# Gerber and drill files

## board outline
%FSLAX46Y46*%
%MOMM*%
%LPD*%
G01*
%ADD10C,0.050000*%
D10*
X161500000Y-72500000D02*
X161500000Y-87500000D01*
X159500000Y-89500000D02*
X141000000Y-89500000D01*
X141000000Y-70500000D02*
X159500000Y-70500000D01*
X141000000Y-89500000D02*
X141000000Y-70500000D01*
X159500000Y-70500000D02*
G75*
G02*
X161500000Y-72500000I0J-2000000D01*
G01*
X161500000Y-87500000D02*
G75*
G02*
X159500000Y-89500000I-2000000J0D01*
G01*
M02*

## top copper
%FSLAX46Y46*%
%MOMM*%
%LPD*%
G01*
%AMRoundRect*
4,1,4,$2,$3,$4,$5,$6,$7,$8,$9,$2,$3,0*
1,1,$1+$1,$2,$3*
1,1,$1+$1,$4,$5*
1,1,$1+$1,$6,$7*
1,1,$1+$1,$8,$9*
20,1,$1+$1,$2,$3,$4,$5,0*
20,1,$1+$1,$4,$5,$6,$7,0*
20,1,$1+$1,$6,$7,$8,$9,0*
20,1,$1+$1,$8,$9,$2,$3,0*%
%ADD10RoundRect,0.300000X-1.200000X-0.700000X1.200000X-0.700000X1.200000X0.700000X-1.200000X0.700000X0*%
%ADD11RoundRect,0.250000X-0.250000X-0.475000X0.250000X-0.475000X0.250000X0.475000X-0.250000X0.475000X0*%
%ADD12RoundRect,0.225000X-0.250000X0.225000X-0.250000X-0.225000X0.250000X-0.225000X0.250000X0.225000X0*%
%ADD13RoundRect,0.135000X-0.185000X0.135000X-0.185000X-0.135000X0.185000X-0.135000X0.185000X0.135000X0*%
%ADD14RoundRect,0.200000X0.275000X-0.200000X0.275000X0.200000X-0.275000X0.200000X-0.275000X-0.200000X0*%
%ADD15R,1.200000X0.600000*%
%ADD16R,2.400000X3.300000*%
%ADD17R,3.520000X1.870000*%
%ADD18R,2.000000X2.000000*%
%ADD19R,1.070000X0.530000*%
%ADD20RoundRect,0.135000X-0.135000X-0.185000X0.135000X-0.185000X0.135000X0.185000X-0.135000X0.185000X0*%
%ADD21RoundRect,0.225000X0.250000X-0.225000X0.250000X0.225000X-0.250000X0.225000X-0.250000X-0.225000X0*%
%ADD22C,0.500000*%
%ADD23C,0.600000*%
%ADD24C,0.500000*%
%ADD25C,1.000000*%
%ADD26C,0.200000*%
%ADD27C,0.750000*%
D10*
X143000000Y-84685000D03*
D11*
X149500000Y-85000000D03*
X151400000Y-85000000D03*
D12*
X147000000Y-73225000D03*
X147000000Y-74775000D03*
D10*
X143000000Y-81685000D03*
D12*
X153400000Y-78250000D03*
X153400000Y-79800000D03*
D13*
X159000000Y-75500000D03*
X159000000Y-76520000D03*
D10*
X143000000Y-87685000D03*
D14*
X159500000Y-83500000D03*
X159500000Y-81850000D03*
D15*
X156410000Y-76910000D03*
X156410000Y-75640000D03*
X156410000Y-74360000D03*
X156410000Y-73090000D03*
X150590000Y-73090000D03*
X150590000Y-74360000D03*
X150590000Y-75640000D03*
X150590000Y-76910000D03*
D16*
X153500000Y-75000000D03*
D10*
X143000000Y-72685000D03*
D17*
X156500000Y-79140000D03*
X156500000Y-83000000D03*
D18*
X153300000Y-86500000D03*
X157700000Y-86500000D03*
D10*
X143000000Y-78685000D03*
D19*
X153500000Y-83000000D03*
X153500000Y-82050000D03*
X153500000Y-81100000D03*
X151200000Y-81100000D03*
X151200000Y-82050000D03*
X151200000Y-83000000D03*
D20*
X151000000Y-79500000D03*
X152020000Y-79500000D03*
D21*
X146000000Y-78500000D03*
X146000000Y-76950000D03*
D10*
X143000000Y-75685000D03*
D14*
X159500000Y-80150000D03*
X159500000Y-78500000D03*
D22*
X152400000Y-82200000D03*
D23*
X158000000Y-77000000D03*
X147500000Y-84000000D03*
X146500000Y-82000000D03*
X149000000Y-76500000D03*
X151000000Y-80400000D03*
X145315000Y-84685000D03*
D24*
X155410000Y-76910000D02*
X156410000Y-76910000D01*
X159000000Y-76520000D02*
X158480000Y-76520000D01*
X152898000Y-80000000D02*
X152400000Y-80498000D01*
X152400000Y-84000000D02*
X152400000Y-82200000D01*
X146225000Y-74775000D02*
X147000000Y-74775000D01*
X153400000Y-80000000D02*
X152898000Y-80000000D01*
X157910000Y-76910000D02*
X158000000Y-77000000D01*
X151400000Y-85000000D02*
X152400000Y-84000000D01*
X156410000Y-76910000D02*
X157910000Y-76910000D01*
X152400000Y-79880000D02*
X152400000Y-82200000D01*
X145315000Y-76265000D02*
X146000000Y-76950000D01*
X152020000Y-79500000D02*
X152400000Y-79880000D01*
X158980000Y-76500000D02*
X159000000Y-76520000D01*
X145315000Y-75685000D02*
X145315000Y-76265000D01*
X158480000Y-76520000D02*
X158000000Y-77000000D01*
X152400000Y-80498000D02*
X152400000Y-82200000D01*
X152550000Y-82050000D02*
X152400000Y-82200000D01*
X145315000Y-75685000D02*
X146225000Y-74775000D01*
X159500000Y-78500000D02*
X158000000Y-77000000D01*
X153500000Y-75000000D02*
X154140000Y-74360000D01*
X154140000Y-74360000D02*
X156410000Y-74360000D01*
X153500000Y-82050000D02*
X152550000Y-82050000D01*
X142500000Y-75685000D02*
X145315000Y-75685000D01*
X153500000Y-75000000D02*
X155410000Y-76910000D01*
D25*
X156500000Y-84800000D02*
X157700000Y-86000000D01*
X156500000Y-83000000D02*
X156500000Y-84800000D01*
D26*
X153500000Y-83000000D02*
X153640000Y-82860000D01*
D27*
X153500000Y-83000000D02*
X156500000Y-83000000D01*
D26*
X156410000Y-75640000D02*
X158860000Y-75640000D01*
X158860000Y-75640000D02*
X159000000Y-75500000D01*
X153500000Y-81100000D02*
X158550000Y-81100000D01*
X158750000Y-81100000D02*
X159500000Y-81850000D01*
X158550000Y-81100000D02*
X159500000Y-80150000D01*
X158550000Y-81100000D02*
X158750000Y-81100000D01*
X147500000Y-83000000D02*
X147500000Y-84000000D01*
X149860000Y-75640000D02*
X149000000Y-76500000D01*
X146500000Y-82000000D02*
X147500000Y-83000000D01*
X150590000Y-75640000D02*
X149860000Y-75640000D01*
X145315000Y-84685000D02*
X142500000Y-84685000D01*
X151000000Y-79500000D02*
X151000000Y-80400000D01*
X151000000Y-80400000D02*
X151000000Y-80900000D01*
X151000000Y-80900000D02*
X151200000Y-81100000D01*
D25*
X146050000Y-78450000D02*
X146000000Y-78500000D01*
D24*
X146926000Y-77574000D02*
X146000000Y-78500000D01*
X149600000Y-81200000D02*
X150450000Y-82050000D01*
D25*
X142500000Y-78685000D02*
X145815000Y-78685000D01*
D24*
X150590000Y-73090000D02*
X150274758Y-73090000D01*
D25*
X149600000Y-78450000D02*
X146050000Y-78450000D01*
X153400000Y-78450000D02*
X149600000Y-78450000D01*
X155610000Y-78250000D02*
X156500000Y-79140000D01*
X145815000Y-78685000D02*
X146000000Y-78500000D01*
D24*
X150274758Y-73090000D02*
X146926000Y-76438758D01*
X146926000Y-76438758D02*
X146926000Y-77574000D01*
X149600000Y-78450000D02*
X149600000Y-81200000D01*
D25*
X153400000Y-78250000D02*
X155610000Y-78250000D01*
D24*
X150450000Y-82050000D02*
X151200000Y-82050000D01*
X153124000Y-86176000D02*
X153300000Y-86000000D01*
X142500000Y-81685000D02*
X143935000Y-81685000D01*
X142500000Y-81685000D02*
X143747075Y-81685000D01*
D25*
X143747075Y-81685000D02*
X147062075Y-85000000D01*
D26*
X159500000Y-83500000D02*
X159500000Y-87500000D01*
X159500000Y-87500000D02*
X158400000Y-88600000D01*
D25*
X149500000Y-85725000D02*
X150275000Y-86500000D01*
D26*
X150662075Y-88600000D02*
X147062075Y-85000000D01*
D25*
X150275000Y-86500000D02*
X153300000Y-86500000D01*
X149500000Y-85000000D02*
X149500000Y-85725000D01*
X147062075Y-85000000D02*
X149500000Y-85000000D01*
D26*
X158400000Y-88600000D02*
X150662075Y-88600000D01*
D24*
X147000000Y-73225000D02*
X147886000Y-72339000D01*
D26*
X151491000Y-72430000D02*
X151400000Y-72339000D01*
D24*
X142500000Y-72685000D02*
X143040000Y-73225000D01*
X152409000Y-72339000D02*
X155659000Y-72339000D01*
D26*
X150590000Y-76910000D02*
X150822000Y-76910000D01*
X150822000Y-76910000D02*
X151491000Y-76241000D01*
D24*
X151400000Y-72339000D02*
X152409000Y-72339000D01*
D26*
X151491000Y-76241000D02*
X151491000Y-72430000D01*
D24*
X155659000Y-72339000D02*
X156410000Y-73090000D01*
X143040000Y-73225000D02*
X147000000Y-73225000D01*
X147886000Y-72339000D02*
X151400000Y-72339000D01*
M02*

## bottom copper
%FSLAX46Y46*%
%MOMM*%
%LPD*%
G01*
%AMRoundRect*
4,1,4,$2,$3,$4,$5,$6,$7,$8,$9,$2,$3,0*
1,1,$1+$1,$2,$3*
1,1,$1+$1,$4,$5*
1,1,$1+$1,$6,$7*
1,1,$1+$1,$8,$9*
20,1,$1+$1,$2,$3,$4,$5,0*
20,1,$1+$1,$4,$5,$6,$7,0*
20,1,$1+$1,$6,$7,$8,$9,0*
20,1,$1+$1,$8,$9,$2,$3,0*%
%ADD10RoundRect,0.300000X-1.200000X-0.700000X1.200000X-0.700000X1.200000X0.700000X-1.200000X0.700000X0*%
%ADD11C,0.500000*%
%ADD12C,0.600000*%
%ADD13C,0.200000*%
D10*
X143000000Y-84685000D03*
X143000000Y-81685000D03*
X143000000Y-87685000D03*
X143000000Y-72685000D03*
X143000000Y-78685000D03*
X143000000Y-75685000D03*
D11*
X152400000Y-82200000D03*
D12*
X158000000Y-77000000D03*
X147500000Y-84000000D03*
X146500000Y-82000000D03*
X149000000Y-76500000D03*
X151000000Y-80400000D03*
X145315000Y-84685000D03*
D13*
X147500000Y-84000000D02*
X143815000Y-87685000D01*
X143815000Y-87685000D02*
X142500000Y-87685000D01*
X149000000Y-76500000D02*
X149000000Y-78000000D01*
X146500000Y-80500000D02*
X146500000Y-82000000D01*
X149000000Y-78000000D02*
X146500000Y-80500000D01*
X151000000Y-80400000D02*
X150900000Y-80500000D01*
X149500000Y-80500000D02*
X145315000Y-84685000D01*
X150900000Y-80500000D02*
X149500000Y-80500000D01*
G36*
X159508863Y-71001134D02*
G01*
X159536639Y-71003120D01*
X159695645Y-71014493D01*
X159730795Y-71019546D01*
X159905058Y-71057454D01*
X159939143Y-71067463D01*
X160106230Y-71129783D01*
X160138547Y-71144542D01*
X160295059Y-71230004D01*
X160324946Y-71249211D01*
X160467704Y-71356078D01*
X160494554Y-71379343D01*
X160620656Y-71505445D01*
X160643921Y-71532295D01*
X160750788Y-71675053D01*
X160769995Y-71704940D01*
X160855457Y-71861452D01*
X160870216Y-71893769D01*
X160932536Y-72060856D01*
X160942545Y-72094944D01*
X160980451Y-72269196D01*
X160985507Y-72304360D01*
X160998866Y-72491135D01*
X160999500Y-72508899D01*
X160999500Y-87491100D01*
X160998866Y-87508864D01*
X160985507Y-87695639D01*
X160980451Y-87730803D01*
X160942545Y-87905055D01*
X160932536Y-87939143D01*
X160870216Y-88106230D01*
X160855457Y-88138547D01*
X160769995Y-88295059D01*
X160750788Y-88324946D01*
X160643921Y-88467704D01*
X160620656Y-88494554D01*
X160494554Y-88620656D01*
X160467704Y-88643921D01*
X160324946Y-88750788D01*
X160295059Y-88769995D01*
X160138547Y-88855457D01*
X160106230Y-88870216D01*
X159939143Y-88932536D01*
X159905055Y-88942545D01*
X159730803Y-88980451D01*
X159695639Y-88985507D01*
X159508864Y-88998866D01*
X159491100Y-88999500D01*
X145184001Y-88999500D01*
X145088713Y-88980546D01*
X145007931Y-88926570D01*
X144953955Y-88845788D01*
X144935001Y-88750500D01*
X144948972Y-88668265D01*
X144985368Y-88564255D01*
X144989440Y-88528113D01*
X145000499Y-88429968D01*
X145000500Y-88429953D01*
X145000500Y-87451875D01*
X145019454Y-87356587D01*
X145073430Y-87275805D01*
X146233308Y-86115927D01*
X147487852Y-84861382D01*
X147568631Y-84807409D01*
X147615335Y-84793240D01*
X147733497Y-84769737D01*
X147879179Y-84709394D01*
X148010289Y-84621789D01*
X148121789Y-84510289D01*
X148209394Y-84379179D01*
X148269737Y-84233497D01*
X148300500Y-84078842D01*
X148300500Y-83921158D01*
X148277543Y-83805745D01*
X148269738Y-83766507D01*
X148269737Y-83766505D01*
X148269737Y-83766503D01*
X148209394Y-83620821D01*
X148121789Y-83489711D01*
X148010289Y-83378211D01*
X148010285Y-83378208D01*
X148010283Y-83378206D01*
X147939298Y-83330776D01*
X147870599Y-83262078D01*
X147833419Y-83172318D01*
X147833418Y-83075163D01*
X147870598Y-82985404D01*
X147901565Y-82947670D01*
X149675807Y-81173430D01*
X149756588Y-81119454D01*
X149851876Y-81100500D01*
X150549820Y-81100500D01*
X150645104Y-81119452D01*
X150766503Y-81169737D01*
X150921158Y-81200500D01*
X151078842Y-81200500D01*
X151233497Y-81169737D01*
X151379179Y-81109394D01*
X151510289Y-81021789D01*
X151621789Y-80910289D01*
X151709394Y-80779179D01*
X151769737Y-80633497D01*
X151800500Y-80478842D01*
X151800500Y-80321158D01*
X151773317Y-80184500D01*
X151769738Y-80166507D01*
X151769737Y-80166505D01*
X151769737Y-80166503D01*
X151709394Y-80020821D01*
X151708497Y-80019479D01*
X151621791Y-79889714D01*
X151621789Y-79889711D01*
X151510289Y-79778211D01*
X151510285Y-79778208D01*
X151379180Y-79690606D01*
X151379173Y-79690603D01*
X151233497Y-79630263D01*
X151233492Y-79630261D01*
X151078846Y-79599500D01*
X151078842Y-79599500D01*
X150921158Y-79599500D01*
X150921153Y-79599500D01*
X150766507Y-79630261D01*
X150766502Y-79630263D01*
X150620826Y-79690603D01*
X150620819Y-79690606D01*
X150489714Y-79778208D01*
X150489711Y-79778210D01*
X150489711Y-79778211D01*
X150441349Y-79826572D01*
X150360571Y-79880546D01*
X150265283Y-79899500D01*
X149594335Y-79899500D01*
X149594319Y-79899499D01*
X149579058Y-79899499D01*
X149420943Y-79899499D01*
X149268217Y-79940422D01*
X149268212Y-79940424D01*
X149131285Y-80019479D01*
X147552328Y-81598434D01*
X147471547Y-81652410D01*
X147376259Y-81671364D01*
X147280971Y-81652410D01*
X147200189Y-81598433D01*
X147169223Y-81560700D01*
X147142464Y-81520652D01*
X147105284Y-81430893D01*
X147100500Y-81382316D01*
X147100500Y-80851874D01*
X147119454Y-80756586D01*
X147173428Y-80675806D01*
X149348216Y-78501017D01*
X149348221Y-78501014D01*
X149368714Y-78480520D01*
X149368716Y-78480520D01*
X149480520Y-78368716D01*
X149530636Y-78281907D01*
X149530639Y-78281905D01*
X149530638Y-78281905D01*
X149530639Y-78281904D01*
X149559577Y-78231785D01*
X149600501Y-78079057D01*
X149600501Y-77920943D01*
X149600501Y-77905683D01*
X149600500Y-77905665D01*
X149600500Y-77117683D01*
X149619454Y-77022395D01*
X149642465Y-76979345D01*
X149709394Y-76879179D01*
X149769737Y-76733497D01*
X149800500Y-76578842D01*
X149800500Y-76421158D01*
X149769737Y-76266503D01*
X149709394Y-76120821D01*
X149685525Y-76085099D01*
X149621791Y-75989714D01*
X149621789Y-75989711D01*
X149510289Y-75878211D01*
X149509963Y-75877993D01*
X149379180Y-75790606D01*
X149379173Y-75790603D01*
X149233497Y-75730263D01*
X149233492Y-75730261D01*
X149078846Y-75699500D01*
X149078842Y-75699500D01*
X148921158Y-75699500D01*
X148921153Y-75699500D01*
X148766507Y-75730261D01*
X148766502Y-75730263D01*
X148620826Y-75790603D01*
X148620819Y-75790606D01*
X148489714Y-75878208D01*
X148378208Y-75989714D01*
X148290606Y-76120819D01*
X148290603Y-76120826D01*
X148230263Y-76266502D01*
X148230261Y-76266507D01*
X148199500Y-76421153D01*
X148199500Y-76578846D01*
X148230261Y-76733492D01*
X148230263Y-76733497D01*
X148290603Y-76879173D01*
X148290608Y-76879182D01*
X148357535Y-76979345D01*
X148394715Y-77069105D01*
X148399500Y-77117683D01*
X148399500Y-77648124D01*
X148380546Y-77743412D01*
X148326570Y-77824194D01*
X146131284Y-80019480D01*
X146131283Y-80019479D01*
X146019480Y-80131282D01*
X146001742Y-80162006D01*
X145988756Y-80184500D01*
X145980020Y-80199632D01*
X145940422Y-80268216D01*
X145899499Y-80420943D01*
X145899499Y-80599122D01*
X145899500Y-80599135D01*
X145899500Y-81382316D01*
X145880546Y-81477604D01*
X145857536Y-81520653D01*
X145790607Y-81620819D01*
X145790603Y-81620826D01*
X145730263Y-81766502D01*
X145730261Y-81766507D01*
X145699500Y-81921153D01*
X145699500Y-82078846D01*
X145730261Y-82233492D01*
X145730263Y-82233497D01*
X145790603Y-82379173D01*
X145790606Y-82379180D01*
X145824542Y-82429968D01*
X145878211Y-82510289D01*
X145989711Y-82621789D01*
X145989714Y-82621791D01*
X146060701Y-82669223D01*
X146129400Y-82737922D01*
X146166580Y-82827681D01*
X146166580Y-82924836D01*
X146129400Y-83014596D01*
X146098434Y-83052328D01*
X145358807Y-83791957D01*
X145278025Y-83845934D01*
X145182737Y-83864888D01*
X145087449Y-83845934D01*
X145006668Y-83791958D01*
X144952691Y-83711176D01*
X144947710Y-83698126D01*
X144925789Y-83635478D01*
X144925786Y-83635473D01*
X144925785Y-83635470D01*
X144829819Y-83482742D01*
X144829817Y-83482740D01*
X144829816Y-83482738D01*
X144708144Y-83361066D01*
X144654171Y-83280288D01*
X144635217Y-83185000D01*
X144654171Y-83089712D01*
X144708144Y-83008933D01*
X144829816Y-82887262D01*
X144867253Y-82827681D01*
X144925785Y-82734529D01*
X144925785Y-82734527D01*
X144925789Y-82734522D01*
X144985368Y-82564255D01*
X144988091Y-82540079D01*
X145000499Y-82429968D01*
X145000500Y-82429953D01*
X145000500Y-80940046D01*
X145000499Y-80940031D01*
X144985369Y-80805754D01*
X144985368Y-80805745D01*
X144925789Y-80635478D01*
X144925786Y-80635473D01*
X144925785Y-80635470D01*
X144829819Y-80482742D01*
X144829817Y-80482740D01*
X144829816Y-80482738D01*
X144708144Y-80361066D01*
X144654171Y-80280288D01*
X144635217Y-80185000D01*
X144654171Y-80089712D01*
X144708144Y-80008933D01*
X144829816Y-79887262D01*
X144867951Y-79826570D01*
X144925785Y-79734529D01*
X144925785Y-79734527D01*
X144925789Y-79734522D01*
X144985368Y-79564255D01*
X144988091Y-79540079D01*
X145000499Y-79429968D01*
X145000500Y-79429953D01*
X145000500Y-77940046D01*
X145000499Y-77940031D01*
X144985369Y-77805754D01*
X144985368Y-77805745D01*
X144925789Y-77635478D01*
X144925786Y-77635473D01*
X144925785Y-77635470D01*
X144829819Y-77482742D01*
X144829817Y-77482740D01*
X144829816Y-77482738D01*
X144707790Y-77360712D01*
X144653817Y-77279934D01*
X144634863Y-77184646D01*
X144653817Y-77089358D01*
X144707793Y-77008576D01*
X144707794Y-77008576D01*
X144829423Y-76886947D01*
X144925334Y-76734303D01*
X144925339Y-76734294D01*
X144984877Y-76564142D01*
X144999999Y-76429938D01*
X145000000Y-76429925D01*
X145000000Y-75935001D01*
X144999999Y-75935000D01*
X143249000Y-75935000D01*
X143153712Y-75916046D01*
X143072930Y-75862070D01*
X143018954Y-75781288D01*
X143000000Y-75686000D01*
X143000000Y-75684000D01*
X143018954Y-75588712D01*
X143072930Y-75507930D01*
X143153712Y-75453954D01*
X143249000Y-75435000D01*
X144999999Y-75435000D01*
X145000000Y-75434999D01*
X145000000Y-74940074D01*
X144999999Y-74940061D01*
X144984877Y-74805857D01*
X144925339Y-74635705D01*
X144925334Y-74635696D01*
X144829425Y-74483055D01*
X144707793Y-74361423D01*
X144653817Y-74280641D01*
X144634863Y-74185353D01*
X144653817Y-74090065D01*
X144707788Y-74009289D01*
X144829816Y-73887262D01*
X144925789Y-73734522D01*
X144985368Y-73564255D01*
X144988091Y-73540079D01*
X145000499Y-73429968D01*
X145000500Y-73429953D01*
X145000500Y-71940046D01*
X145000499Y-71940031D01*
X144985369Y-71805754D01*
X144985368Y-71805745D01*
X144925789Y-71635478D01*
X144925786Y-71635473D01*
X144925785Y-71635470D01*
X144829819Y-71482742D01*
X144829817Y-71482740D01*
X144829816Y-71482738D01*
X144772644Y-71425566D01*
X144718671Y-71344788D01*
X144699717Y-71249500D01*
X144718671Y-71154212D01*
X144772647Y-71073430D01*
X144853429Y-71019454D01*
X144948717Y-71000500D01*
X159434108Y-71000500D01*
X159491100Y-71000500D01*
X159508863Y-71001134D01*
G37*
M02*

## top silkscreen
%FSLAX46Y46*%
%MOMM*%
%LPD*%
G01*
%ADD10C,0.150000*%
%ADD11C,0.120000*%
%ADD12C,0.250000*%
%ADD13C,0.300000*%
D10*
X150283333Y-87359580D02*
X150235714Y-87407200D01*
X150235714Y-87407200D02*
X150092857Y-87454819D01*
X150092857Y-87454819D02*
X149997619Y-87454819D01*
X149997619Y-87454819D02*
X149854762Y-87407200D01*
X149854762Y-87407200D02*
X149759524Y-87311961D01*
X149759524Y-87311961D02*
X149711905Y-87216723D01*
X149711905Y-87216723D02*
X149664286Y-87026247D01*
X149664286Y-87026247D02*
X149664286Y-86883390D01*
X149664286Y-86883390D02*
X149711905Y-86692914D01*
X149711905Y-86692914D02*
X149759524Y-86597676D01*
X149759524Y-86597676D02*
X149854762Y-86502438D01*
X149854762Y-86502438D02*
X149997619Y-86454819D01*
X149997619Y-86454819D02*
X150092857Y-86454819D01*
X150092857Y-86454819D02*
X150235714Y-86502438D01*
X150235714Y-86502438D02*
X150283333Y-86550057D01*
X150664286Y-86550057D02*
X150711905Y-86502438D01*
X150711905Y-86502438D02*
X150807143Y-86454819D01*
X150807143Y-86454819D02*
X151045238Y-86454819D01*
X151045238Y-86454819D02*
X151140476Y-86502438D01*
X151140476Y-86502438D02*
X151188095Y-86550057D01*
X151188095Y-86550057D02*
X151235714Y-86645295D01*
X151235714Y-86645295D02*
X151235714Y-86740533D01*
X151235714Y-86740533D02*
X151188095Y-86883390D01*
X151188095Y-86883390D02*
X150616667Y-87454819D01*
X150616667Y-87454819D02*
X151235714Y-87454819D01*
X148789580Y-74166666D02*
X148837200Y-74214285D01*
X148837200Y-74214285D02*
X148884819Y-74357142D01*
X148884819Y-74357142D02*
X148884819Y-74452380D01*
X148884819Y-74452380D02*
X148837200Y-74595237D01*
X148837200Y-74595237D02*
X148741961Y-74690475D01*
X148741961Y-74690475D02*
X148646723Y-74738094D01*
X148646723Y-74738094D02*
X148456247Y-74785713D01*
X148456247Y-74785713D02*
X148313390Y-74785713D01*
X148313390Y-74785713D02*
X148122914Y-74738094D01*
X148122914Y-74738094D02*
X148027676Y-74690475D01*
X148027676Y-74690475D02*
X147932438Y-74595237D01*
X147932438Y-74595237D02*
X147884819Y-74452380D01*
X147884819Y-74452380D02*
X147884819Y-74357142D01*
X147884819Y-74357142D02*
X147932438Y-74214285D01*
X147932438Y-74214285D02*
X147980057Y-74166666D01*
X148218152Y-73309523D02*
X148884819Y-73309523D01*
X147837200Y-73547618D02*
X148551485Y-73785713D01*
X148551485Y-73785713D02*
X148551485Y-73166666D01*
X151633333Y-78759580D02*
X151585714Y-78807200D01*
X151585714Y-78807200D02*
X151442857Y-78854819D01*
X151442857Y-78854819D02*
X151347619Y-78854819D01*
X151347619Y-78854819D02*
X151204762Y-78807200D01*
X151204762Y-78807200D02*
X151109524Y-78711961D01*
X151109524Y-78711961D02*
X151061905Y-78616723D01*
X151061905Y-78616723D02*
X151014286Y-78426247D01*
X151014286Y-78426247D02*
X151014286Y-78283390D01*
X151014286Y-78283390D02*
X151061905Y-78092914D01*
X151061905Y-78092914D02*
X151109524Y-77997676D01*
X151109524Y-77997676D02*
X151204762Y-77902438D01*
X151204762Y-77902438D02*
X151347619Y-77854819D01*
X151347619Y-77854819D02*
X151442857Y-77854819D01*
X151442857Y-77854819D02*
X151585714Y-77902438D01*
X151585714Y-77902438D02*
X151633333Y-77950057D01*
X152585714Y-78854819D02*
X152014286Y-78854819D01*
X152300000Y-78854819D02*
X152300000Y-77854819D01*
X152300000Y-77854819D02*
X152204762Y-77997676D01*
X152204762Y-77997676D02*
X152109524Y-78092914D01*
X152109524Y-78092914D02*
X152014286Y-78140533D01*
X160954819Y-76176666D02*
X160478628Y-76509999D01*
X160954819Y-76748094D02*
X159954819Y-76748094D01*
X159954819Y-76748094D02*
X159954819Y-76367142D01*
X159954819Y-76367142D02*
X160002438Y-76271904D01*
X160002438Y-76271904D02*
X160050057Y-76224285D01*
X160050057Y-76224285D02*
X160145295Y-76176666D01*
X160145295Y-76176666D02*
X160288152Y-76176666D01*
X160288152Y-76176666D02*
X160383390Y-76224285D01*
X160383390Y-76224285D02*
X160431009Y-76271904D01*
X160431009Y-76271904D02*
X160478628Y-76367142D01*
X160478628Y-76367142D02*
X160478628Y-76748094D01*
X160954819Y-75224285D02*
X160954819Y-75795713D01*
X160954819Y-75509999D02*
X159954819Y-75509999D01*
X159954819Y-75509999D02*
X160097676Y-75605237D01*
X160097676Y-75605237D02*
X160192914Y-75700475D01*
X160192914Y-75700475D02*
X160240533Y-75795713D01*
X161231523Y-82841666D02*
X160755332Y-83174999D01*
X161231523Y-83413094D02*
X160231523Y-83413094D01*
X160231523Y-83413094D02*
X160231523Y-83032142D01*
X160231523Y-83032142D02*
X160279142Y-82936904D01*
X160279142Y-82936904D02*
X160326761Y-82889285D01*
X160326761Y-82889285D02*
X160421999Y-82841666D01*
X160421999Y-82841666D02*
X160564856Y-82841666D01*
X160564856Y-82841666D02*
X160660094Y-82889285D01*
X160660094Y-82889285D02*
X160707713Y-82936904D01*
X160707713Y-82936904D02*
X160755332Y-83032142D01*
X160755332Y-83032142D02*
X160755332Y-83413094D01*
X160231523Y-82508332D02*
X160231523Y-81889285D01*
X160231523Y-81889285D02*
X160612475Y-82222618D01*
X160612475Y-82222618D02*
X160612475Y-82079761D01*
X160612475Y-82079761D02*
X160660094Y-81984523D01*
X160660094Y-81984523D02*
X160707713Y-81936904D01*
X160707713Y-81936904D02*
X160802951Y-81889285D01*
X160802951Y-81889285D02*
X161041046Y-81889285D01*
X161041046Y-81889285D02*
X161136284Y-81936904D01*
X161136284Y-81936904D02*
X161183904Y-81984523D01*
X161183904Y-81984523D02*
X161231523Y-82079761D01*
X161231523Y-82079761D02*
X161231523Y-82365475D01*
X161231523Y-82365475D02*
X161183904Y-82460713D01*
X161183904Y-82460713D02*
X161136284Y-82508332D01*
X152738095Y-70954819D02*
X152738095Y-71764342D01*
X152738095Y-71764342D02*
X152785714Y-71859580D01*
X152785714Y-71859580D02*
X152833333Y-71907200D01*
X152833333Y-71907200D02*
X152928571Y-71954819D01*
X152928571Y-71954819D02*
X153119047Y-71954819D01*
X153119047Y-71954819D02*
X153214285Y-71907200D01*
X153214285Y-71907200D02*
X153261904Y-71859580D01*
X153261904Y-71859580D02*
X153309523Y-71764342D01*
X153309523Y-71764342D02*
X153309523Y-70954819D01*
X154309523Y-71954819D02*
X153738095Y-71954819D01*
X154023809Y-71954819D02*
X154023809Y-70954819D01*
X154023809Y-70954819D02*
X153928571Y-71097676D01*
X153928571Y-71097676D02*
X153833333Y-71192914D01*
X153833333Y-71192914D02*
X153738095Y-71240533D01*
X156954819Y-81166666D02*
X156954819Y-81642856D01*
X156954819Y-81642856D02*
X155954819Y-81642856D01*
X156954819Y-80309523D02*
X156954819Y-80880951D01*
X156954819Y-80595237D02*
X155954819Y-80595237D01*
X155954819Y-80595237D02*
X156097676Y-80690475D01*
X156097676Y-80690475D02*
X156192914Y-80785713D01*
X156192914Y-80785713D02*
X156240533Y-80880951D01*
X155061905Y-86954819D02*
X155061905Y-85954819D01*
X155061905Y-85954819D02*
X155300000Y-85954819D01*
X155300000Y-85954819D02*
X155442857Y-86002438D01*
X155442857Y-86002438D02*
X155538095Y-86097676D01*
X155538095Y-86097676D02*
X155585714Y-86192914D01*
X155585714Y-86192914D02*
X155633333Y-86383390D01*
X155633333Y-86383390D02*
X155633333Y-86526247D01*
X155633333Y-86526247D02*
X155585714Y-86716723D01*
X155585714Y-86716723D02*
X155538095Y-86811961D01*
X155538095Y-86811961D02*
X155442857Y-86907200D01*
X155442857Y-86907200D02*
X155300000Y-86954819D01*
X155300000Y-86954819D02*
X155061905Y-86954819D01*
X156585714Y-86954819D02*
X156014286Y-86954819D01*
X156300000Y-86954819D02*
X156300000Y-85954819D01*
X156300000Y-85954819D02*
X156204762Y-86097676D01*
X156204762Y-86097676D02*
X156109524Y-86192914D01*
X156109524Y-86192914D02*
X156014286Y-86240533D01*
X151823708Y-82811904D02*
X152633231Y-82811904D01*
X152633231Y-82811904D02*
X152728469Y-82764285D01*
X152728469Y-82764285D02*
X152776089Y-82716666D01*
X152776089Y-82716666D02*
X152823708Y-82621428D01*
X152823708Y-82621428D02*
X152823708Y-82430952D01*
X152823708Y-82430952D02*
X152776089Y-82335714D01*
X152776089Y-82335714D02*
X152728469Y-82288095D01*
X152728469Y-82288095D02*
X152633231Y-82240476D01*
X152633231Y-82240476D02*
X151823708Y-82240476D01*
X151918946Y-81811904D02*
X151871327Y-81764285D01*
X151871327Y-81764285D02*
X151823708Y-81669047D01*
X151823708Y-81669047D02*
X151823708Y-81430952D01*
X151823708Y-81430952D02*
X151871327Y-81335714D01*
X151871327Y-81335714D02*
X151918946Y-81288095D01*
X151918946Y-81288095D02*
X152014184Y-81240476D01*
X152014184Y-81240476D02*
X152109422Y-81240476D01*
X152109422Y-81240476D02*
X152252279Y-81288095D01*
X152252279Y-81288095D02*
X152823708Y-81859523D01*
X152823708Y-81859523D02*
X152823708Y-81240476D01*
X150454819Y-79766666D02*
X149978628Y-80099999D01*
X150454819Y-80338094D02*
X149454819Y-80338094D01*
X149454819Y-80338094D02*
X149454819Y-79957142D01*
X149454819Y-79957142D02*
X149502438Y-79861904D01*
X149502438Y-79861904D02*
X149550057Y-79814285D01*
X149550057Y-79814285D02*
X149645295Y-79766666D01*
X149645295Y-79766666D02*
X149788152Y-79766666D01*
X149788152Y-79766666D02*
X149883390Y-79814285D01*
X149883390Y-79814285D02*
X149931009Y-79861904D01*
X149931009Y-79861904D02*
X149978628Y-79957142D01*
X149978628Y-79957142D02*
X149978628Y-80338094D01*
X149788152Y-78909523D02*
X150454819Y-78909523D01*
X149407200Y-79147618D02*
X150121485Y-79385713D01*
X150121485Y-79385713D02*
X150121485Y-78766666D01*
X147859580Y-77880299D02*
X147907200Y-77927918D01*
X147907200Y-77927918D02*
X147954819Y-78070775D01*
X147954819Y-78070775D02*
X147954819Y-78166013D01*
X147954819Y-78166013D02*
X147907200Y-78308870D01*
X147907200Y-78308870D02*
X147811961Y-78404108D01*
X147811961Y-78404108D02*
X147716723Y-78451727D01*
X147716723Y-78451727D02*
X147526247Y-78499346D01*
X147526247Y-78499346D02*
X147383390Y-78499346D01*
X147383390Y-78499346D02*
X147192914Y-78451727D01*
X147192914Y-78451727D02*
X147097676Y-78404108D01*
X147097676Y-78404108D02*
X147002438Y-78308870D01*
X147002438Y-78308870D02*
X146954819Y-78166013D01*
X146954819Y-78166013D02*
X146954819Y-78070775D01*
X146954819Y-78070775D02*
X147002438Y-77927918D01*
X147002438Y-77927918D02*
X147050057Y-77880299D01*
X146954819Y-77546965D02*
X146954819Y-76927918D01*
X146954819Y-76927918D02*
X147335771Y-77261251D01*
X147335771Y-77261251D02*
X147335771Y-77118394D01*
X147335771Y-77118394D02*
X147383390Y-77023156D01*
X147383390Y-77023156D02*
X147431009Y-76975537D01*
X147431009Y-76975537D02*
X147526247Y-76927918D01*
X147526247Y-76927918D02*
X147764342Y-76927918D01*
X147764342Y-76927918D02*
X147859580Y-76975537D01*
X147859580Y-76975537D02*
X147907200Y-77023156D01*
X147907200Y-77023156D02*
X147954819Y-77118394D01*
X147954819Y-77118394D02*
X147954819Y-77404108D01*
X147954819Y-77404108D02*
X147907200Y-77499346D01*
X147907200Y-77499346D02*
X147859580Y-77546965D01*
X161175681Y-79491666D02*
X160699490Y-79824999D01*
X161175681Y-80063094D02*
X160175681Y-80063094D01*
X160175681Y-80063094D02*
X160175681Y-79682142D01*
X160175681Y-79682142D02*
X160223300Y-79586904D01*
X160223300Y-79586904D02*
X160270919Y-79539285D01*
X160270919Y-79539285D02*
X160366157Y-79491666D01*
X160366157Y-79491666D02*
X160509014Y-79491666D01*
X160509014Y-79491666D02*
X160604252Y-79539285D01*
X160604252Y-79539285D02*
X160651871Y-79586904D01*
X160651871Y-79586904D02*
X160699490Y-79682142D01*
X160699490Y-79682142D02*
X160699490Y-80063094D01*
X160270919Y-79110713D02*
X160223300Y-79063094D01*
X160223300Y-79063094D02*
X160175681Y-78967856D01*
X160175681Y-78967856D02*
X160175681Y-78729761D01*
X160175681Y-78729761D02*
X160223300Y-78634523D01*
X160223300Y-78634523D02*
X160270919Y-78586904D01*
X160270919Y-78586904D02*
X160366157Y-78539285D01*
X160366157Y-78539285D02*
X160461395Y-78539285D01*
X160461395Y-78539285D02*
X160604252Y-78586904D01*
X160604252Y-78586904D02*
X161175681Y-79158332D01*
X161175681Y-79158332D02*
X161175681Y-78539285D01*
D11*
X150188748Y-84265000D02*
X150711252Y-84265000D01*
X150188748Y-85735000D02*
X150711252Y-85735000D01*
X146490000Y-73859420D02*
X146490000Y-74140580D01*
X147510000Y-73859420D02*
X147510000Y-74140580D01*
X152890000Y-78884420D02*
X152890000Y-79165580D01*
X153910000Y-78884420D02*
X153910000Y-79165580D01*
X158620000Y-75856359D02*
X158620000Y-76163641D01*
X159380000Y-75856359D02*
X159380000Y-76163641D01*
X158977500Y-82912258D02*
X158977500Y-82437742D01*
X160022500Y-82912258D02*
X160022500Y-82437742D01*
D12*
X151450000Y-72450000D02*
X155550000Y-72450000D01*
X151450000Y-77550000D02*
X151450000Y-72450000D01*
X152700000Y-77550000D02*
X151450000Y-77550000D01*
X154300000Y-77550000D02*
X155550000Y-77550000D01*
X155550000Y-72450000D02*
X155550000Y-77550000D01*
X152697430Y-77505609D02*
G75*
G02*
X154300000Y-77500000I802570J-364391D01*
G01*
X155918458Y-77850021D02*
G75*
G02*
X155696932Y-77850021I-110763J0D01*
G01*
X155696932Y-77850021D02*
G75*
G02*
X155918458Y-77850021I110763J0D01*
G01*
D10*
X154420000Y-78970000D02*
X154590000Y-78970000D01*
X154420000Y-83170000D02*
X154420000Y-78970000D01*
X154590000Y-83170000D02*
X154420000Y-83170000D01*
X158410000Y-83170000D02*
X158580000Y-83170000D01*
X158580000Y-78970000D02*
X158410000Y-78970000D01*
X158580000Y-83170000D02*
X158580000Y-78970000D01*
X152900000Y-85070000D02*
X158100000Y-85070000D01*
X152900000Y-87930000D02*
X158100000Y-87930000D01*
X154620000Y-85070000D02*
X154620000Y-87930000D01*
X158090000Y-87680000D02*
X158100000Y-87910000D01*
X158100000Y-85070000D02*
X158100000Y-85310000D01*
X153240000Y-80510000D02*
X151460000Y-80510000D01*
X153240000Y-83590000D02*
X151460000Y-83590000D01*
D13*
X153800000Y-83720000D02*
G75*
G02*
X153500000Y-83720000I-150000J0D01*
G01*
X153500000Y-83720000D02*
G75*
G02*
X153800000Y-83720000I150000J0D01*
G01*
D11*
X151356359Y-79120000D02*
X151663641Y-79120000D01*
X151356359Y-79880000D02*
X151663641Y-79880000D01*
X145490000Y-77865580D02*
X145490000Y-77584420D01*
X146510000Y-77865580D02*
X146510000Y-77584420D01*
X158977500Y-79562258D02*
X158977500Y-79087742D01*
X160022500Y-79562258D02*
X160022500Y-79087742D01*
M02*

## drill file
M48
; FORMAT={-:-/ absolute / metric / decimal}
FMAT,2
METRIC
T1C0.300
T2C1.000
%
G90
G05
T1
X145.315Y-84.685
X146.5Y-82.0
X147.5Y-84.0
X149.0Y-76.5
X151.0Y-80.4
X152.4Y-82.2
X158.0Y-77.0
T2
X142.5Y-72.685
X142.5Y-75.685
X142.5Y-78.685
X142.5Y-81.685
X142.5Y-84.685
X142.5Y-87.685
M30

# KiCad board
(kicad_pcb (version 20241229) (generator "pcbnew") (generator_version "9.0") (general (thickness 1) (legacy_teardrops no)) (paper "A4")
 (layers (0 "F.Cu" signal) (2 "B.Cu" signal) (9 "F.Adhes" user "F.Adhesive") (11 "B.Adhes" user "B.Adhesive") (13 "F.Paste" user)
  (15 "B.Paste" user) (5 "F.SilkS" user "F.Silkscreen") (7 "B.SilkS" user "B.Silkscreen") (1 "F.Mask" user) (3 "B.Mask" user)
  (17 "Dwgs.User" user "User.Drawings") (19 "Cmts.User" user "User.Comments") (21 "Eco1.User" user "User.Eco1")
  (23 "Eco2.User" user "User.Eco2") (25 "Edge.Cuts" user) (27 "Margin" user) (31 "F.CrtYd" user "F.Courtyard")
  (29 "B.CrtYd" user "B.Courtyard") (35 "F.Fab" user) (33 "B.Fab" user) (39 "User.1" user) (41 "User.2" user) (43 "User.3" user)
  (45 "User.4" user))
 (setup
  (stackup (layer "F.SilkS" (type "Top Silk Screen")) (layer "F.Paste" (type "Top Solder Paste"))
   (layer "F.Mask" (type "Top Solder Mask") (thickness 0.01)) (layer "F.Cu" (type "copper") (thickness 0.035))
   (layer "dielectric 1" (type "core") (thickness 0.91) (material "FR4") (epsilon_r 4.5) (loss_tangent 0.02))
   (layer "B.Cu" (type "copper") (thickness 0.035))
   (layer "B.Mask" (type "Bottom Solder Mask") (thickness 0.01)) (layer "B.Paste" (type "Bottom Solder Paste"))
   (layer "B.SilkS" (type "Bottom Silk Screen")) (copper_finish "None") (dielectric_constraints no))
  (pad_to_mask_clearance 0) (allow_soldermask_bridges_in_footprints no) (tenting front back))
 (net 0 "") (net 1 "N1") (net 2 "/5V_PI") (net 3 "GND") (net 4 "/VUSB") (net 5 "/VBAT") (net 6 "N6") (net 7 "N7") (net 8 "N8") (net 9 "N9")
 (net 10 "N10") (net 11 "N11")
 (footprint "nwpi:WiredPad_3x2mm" (layer "F.Cu") (at 142.5 84.685)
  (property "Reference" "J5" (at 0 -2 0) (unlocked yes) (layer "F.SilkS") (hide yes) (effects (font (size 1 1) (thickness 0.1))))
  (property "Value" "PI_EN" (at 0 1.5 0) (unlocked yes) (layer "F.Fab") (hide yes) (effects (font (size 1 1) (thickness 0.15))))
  (pad "1" thru_hole roundrect (at 0 0) (size 3 2) (drill 1 (offset 0.5 0)) (layers "*.Cu" "*.Mask") (remove_unused_layers no)
   (roundrect_rratio 0.15) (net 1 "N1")))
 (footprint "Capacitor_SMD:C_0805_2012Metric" (layer "F.Cu") (at 150.45 85)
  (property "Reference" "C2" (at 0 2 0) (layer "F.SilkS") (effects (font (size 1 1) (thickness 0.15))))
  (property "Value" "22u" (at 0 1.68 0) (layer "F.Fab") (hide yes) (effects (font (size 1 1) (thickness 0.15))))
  (fp_line (start -0.261252 -0.735) (end 0.261252 -0.735) (stroke (width 0.12) (type solid)) (layer "F.SilkS"))
  (fp_line (start -0.261252 0.735) (end 0.261252 0.735) (stroke (width 0.12) (type solid)) (layer "F.SilkS"))
  (pad "1" smd roundrect (at -0.95 0) (size 1 1.45) (layers "F.Cu" "F.Mask" "F.Paste") (roundrect_rratio 0.25) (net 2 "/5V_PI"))
  (pad "2" smd roundrect (at 0.95 0) (size 1 1.45) (layers "F.Cu" "F.Mask" "F.Paste") (roundrect_rratio 0.25) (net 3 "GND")))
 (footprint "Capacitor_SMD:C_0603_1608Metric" (layer "F.Cu") (at 147 74 -90)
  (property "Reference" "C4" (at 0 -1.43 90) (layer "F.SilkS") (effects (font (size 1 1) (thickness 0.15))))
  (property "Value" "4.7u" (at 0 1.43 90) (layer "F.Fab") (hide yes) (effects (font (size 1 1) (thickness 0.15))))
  (fp_line (start -0.14058 0.51) (end 0.14058 0.51) (stroke (width 0.12) (type solid)) (layer "F.SilkS"))
  (fp_line (start -0.14058 -0.51) (end 0.14058 -0.51) (stroke (width 0.12) (type solid)) (layer "F.SilkS"))
  (pad "1" smd roundrect (at -0.775 0 270) (size 0.9 0.95) (layers "F.Cu" "F.Mask" "F.Paste") (roundrect_rratio 0.25) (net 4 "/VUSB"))
  (pad "2" smd roundrect (at 0.775 0 270) (size 0.9 0.95) (layers "F.Cu" "F.Mask" "F.Paste") (roundrect_rratio 0.25) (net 3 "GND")))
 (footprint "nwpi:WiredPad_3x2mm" (layer "F.Cu") (at 142.5 81.685)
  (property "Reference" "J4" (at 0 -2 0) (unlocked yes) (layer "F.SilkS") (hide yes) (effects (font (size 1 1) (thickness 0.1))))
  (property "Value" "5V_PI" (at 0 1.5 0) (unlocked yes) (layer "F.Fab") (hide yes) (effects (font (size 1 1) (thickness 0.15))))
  (pad "1" thru_hole roundrect (at 0 0) (size 3 2) (drill 1 (offset 0.5 0)) (layers "*.Cu" "*.Mask") (remove_unused_layers no)
   (roundrect_rratio 0.15) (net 2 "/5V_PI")))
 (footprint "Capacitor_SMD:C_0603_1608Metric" (layer "F.Cu") (at 153.4 79.025 -90)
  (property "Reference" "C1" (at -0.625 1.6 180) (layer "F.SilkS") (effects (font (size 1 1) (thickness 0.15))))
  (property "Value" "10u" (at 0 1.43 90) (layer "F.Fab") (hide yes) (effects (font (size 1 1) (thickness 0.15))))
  (fp_line (start -0.14058 0.51) (end 0.14058 0.51) (stroke (width 0.12) (type solid)) (layer "F.SilkS"))
  (fp_line (start -0.14058 -0.51) (end 0.14058 -0.51) (stroke (width 0.12) (type solid)) (layer "F.SilkS"))
  (pad "1" smd roundrect (at -0.775 0 270) (size 0.9 0.95) (layers "F.Cu" "F.Mask" "F.Paste") (roundrect_rratio 0.25) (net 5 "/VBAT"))
  (pad "2" smd roundrect (at 0.775 0 270) (size 0.9 0.95) (layers "F.Cu" "F.Mask" "F.Paste") (roundrect_rratio 0.25) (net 3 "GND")))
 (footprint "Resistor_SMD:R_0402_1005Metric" (layer "F.Cu") (at 159 76.01 -90)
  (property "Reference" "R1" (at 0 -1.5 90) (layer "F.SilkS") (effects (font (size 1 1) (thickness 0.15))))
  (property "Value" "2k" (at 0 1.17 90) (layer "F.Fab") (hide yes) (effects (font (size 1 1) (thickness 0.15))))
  (fp_line (start -0.153641 0.38) (end 0.153641 0.38) (stroke (width 0.12) (type solid)) (layer "F.SilkS"))
  (fp_line (start -0.153641 -0.38) (end 0.153641 -0.38) (stroke (width 0.12) (type solid)) (layer "F.SilkS"))
  (pad "1" smd roundrect (at -0.51 0 270) (size 0.54 0.64) (layers "F.Cu" "F.Mask" "F.Paste") (roundrect_rratio 0.25) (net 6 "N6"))
  (pad "2" smd roundrect (at 0.51 0 270) (size 0.54 0.64) (layers "F.Cu" "F.Mask" "F.Paste") (roundrect_rratio 0.25) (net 3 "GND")))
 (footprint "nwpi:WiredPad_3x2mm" (layer "F.Cu") (at 142.5 87.685)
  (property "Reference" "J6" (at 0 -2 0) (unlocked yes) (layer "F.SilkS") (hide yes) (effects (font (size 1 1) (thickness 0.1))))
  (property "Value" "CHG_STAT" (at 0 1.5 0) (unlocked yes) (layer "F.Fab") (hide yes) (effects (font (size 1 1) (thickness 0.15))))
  (pad "1" thru_hole roundrect (at 0 0) (size 3 2) (drill 1 (offset 0.5 0)) (layers "*.Cu" "*.Mask") (remove_unused_layers no)
   (roundrect_rratio 0.15) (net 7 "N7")))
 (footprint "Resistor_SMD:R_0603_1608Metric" (layer "F.Cu") (at 159.5 82.675 90)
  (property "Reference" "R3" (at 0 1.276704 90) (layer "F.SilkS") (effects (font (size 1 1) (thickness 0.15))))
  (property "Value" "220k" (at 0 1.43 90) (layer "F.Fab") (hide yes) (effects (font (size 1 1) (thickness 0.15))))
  (fp_line (start -0.237258 -0.5225) (end 0.237258 -0.5225) (stroke (width 0.12) (type solid)) (layer "F.SilkS"))
  (fp_line (start -0.237258 0.5225) (end 0.237258 0.5225) (stroke (width 0.12) (type solid)) (layer "F.SilkS"))
  (pad "1" smd roundrect (at -0.825 0 90) (size 0.8 0.95) (layers "F.Cu" "F.Mask" "F.Paste") (roundrect_rratio 0.25) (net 2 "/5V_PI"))
  (pad "2" smd roundrect (at 0.825 0 90) (size 0.8 0.95) (layers "F.Cu" "F.Mask" "F.Paste") (roundrect_rratio 0.25) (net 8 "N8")))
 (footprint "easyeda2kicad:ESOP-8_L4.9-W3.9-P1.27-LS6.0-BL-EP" (layer "F.Cu") (at 153.5 75 90)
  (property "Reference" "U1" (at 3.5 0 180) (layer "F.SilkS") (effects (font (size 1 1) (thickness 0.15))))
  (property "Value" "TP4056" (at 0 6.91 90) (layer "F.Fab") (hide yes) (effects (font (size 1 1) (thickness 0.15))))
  (fp_line (start 2.55 -2.05) (end 2.55 2.05) (stroke (width 0.25) (type solid)) (layer "F.SilkS"))
  (fp_line (start -2.55 -2.05) (end 2.55 -2.05) (stroke (width 0.25) (type solid)) (layer "F.SilkS"))
  (fp_line (start -2.55 -0.8) (end -2.55 -2.05) (stroke (width 0.25) (type solid)) (layer "F.SilkS"))
  (fp_line (start -2.55 0.8) (end -2.55 2.05) (stroke (width 0.25) (type solid)) (layer "F.SilkS"))
  (fp_line (start 2.55 2.05) (end -2.55 2.05) (stroke (width 0.25) (type solid)) (layer "F.SilkS"))
  (fp_arc (start -2.505609 -0.80257) (mid -1.988586 -0.003085) (end -2.5 0.8) (stroke (width 0.25) (type solid)) (layer "F.SilkS"))
  (fp_circle (center -2.850021 2.307695) (end -2.739258 2.307695) (stroke (width 0.25) (type solid)) (fill no) (layer "F.SilkS"))
  (pad "1" smd rect (at -1.91 2.91 90) (size 0.6 1.2) (layers "F.Cu" "F.Mask" "F.Paste") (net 3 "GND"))
  (pad "2" smd rect (at -0.64 2.91 90) (size 0.6 1.2) (layers "F.Cu" "F.Mask" "F.Paste") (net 6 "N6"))
  (pad "3" smd rect (at 0.64 2.91 90) (size 0.6 1.2) (layers "F.Cu" "F.Mask" "F.Paste") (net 3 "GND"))
  (pad "4" smd rect (at 1.91 2.91 90) (size 0.6 1.2) (layers "F.Cu" "F.Mask" "F.Paste") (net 4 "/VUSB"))
  (pad "5" smd rect (at 1.91 -2.91 90) (size 0.6 1.2) (layers "F.Cu" "F.Mask" "F.Paste") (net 5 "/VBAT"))
  (pad "6" smd rect (at 0.64 -2.91 90) (size 0.6 1.2) (layers "F.Cu" "F.Mask" "F.Paste") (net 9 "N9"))
  (pad "7" smd rect (at -0.64 -2.91 90) (size 0.6 1.2) (layers "F.Cu" "F.Mask" "F.Paste") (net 7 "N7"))
  (pad "8" smd rect (at -1.91 -2.91 90) (size 0.6 1.2) (layers "F.Cu" "F.Mask" "F.Paste") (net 4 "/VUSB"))
  (pad "9" smd rect (at 0 0 270) (size 3.3 2.4) (layers "F.Cu" "F.Mask" "F.Paste") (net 3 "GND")))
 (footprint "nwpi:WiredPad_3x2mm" (layer "F.Cu") (at 142.5 72.685)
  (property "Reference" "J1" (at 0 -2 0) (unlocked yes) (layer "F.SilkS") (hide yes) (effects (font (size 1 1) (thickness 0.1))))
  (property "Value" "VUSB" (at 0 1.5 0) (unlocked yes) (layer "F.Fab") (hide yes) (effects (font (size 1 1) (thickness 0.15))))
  (pad "1" thru_hole roundrect (at 0 0) (size 3 2) (drill 1 (offset 0.5 0)) (layers "*.Cu" "*.Mask") (remove_unused_layers no)
   (roundrect_rratio 0.15) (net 4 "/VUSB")))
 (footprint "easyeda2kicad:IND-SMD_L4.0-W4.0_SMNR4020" (layer "F.Cu") (at 156.5 81.07 90)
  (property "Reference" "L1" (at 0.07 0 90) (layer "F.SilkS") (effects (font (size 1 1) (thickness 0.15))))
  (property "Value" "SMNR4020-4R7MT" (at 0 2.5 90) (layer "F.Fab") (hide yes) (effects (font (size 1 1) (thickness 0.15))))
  (fp_line (start 2.1 -2.08) (end 2.1 -1.91) (stroke (width 0.15) (type solid)) (layer "F.SilkS"))
  (fp_line (start -2.1 -2.08) (end 2.1 -2.08) (stroke (width 0.15) (type solid)) (layer "F.SilkS"))
  (fp_line (start -2.1 -1.91) (end -2.1 -2.08) (stroke (width 0.15) (type solid)) (layer "F.SilkS"))
  (fp_line (start -2.1 1.91) (end -2.1 2.08) (stroke (width 0.15) (type solid)) (layer "F.SilkS"))
  (fp_line (start 2.1 2.08) (end 2.1 1.91) (stroke (width 0.15) (type solid)) (layer "F.SilkS"))
  (fp_line (start -2.1 2.08) (end 2.1 2.08) (stroke (width 0.15) (type solid)) (layer "F.SilkS"))
  (pad "1" smd rect (at 1.93 0 90) (size 1.87 3.52) (layers "F.Cu" "F.Mask" "F.Paste") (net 5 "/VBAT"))
  (pad "2" smd rect (at -1.93 0 90) (size 1.87 3.52) (layers "F.Cu" "F.Mask" "F.Paste") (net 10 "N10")))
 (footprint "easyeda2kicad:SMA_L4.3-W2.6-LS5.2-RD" (layer "F.Cu") (at 155.5 86.5)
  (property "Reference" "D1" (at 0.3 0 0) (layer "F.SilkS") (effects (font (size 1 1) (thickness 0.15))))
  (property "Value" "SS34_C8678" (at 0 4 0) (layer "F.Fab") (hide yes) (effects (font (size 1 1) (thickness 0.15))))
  (fp_line (start -2.6 -1.43) (end 2.6 -1.43) (stroke (width 0.15) (type solid)) (layer "F.SilkS"))
  (fp_line (start -2.6 1.43) (end 2.6 1.43) (stroke (width 0.15) (type solid)) (layer "F.SilkS"))
  (fp_line (start -0.88 -1.43) (end -0.88 1.43) (stroke (width 0.15) (type solid)) (layer "F.SilkS"))
  (fp_line (start 2.59 1.18) (end 2.6 1.41) (stroke (width 0.15) (type solid)) (layer "F.SilkS"))
  (fp_line (start 2.6 -1.43) (end 2.6 -1.19) (stroke (width 0.15) (type solid)) (layer "F.SilkS"))
  (pad "1" smd rect (at -2.2 0 180) (size 2 2) (layers "F.Cu" "F.Mask" "F.Paste") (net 2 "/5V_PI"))
  (pad "2" smd rect (at 2.2 0 180) (size 2 2) (layers "F.Cu" "F.Mask" "F.Paste") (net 10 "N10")))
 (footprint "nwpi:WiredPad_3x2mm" (layer "F.Cu") (at 142.5 78.685)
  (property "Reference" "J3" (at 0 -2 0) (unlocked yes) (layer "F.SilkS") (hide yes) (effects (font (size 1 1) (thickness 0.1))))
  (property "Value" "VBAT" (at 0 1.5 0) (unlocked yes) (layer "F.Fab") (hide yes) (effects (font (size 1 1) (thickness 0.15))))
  (pad "1" thru_hole roundrect (at 0 0) (size 3 2) (drill 1 (offset 0.5 0)) (layers "*.Cu" "*.Mask") (remove_unused_layers no)
   (roundrect_rratio 0.15) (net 5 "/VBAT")))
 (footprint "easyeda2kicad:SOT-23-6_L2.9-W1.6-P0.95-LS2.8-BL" (layer "F.Cu") (at 152.35 82.05 90)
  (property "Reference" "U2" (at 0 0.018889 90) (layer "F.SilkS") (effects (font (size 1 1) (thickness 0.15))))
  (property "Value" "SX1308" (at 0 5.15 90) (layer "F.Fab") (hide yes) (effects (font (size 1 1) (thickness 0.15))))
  (fp_line (start 1.54 0.89) (end 1.54 -0.89) (stroke (width 0.15) (type solid)) (layer "F.SilkS"))
  (fp_line (start -1.54 0.89) (end -1.54 -0.89) (stroke (width 0.15) (type solid)) (layer "F.SilkS"))
  (fp_circle (center -1.67 1.3) (end -1.52 1.3) (stroke (width 0.3) (type solid)) (fill no) (layer "F.SilkS"))
  (pad "1" smd rect (at -0.95 1.15 90) (size 0.53 1.07) (layers "F.Cu" "F.Mask" "F.Paste") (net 10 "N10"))
  (pad "2" smd rect (at 0 1.15 90) (size 0.53 1.07) (layers "F.Cu" "F.Mask" "F.Paste") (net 3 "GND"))
  (pad "3" smd rect (at 0.95 1.15 90) (size 0.53 1.07) (layers "F.Cu" "F.Mask" "F.Paste") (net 8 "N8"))
  (pad "4" smd rect (at 0.95 -1.15 90) (size 0.53 1.07) (layers "F.Cu" "F.Mask" "F.Paste") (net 1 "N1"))
  (pad "5" smd rect (at 0 -1.15 90) (size 0.53 1.07) (layers "F.Cu" "F.Mask" "F.Paste") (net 5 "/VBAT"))
  (pad "6" smd rect (at -0.95 -1.15 90) (size 0.53 1.07) (layers "F.Cu" "F.Mask" "F.Paste") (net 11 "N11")))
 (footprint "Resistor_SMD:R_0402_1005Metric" (layer "F.Cu") (at 151.51 79.5)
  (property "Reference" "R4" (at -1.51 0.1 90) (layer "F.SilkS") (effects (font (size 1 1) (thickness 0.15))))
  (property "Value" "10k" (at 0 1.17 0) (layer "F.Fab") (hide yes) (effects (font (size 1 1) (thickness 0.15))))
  (fp_line (start -0.153641 -0.38) (end 0.153641 -0.38) (stroke (width 0.12) (type solid)) (layer "F.SilkS"))
  (fp_line (start -0.153641 0.38) (end 0.153641 0.38) (stroke (width 0.12) (type solid)) (layer "F.SilkS"))
  (pad "1" smd roundrect (at -0.51 0) (size 0.54 0.64) (layers "F.Cu" "F.Mask" "F.Paste") (roundrect_rratio 0.25) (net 1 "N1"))
  (pad "2" smd roundrect (at 0.51 0) (size 0.54 0.64) (layers "F.Cu" "F.Mask" "F.Paste") (roundrect_rratio 0.25) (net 3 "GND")))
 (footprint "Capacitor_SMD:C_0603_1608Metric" (layer "F.Cu") (at 146 77.725 90)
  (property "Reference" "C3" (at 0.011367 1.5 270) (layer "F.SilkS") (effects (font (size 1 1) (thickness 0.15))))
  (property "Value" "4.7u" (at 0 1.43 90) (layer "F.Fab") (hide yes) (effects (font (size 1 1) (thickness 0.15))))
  (fp_line (start -0.14058 -0.51) (end 0.14058 -0.51) (stroke (width 0.12) (type solid)) (layer "F.SilkS"))
  (fp_line (start -0.14058 0.51) (end 0.14058 0.51) (stroke (width 0.12) (type solid)) (layer "F.SilkS"))
  (pad "1" smd roundrect (at -0.775 0 90) (size 0.9 0.95) (layers "F.Cu" "F.Mask" "F.Paste") (roundrect_rratio 0.25) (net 5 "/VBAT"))
  (pad "2" smd roundrect (at 0.775 0 90) (size 0.9 0.95) (layers "F.Cu" "F.Mask" "F.Paste") (roundrect_rratio 0.25) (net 3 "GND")))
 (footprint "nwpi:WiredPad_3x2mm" (layer "F.Cu") (at 142.5 75.685)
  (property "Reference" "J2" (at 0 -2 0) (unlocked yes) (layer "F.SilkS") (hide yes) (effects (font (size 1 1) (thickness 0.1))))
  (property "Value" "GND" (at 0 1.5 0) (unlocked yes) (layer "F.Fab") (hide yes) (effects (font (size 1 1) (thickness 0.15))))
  (pad "1" thru_hole roundrect (at 0 0) (size 3 2) (drill 1 (offset 0.5 0)) (layers "*.Cu" "*.Mask") (remove_unused_layers no)
   (roundrect_rratio 0.15) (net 3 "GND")))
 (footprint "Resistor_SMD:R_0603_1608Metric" (layer "F.Cu") (at 159.5 79.325 90)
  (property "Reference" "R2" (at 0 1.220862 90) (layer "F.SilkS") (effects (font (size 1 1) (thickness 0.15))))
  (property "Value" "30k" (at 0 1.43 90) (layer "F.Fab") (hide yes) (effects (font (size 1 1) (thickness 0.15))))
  (fp_line (start -0.237258 -0.5225) (end 0.237258 -0.5225) (stroke (width 0.12) (type solid)) (layer "F.SilkS"))
  (fp_line (start -0.237258 0.5225) (end 0.237258 0.5225) (stroke (width 0.12) (type solid)) (layer "F.SilkS"))
  (pad "1" smd roundrect (at -0.825 0 90) (size 0.8 0.95) (layers "F.Cu" "F.Mask" "F.Paste") (roundrect_rratio 0.25) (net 8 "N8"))
  (pad "2" smd roundrect (at 0.825 0 90) (size 0.8 0.95) (layers "F.Cu" "F.Mask" "F.Paste") (roundrect_rratio 0.25) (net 3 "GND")))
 (gr_line (start 161.5 72.5) (end 161.5 87.5) (stroke (width 0.05) (type default)) (layer "Edge.Cuts"))
 (gr_line (start 159.5 89.5) (end 141 89.5) (stroke (width 0.05) (type default)) (layer "Edge.Cuts"))
 (gr_line (start 141 70.5) (end 159.5 70.5) (stroke (width 0.05) (type default)) (layer "Edge.Cuts"))
 (gr_line (start 141 89.5) (end 141 70.5) (stroke (width 0.05) (type default)) (layer "Edge.Cuts"))
 (gr_arc (start 159.5 70.5) (mid 160.914214 71.085786) (end 161.5 72.5) (stroke (width 0.05) (type default)) (layer "Edge.Cuts"))
 (gr_arc (start 161.5 87.5) (mid 160.914214 88.914214) (end 159.5 89.5) (stroke (width 0.05) (type default)) (layer "Edge.Cuts"))
 (segment (start 155.41 76.91) (end 156.41 76.91) (width 0.5) (layer "F.Cu") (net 3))
 (segment (start 159 76.52) (end 158.48 76.52) (width 0.5) (layer "F.Cu") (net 3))
 (segment (start 152.898 80) (end 152.4 80.498) (width 0.5) (layer "F.Cu") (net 3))
 (segment (start 152.4 84) (end 152.4 82.2) (width 0.5) (layer "F.Cu") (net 3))
 (segment (start 146.225 74.775) (end 147 74.775) (width 0.5) (layer "F.Cu") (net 3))
 (segment (start 153.4 80) (end 152.898 80) (width 0.5) (layer "F.Cu") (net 3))
 (segment (start 157.91 76.91) (end 158 77) (width 0.5) (layer "F.Cu") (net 3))
 (segment (start 151.4 85) (end 152.4 84) (width 0.5) (layer "F.Cu") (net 3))
 (segment (start 156.41 76.91) (end 157.91 76.91) (width 0.5) (layer "F.Cu") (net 3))
 (segment (start 152.4 79.88) (end 152.4 82.2) (width 0.5) (layer "F.Cu") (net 3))
 (segment (start 145.315 76.265) (end 146 76.95) (width 0.5) (layer "F.Cu") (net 3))
 (segment (start 152.02 79.5) (end 152.4 79.88) (width 0.5) (layer "F.Cu") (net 3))
 (segment (start 158.98 76.5) (end 159 76.52) (width 0.5) (layer "F.Cu") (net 3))
 (segment (start 145.315 75.685) (end 145.315 76.265) (width 0.5) (layer "F.Cu") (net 3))
 (segment (start 158.48 76.52) (end 158 77) (width 0.5) (layer "F.Cu") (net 3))
 (segment (start 152.4 80.498) (end 152.4 82.2) (width 0.5) (layer "F.Cu") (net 3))
 (segment (start 152.55 82.05) (end 152.4 82.2) (width 0.5) (layer "F.Cu") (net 3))
 (segment (start 145.315 75.685) (end 146.225 74.775) (width 0.5) (layer "F.Cu") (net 3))
 (segment (start 159.5 78.5) (end 158 77) (width 0.5) (layer "F.Cu") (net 3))
 (segment (start 153.5 75) (end 154.14 74.36) (width 0.5) (layer "F.Cu") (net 3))
 (segment (start 154.14 74.36) (end 156.41 74.36) (width 0.5) (layer "F.Cu") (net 3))
 (segment (start 153.5 82.05) (end 152.55 82.05) (width 0.5) (layer "F.Cu") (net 3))
 (segment (start 142.5 75.685) (end 145.315 75.685) (width 0.5) (layer "F.Cu") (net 3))
 (segment (start 153.5 75) (end 155.41 76.91) (width 0.5) (layer "F.Cu") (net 3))
 (via (at 152.4 82.2) (size 0.5) (drill 0.3) (layers "F.Cu" "B.Cu") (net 3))
 (via (at 158 77) (size 0.6) (drill 0.3) (layers "F.Cu" "B.Cu") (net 3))
 (segment (start 156.5 84.8) (end 157.7 86) (width 1) (layer "F.Cu") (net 10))
 (segment (start 156.5 83) (end 156.5 84.8) (width 1) (layer "F.Cu") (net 10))
 (segment (start 153.5 83) (end 153.64 82.86) (width 0.2) (layer "F.Cu") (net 10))
 (segment (start 153.5 83) (end 156.5 83) (width 0.75) (layer "F.Cu") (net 10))
 (segment (start 156.41 75.64) (end 158.86 75.64) (width 0.2) (layer "F.Cu") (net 6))
 (segment (start 158.86 75.64) (end 159 75.5) (width 0.2) (layer "F.Cu") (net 6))
 (segment (start 153.5 81.1) (end 158.55 81.1) (width 0.2) (layer "F.Cu") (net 8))
 (segment (start 158.75 81.1) (end 159.5 81.85) (width 0.2) (layer "F.Cu") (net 8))
 (segment (start 158.55 81.1) (end 159.5 80.15) (width 0.2) (layer "F.Cu") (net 8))
 (segment (start 158.55 81.1) (end 158.75 81.1) (width 0.2) (layer "F.Cu") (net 8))
 (segment (start 147.5 83) (end 147.5 84) (width 0.2) (layer "F.Cu") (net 7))
 (segment (start 149.86 75.64) (end 149 76.5) (width 0.2) (layer "F.Cu") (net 7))
 (segment (start 146.5 82) (end 147.5 83) (width 0.2) (layer "F.Cu") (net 7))
 (segment (start 150.59 75.64) (end 149.86 75.64) (width 0.2) (layer "F.Cu") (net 7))
 (via (at 147.5 84) (size 0.6) (drill 0.3) (layers "F.Cu" "B.Cu") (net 7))
 (via (at 146.5 82) (size 0.6) (drill 0.3) (layers "F.Cu" "B.Cu") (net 7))
 (via (at 149 76.5) (size 0.6) (drill 0.3) (layers "F.Cu" "B.Cu") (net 7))
 (segment (start 147.5 84) (end 143.815 87.685) (width 0.2) (layer "B.Cu") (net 7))
 (segment (start 143.815 87.685) (end 142.5 87.685) (width 0.2) (layer "B.Cu") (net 7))
 (segment (start 149 76.5) (end 149 78) (width 0.2) (layer "B.Cu") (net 7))
 (segment (start 146.5 80.5) (end 146.5 82) (width 0.2) (layer "B.Cu") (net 7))
 (segment (start 149 78) (end 146.5 80.5) (width 0.2) (layer "B.Cu") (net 7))
 (segment (start 145.315 84.685) (end 142.5 84.685) (width 0.2) (layer "F.Cu") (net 1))
 (segment (start 151 79.5) (end 151 80.4) (width 0.2) (layer "F.Cu") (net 1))
 (segment (start 151 80.4) (end 151 80.9) (width 0.2) (layer "F.Cu") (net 1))
 (segment (start 151 80.9) (end 151.2 81.1) (width 0.2) (layer "F.Cu") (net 1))
 (via (at 151 80.4) (size 0.6) (drill 0.3) (layers "F.Cu" "B.Cu") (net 1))
 (via (at 145.315 84.685) (size 0.6) (drill 0.3) (layers "F.Cu" "B.Cu") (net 1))
 (segment (start 151 80.4) (end 150.9 80.5) (width 0.2) (layer "B.Cu") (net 1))
 (segment (start 149.5 80.5) (end 145.315 84.685) (width 0.2) (layer "B.Cu") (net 1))
 (segment (start 150.9 80.5) (end 149.5 80.5) (width 0.2) (layer "B.Cu") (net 1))
 (segment (start 146.05 78.45) (end 146 78.5) (width 1) (layer "F.Cu") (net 5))
 (segment (start 146.926 77.574) (end 146 78.5) (width 0.5) (layer "F.Cu") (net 5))
 (segment (start 149.6 81.2) (end 150.45 82.05) (width 0.5) (layer "F.Cu") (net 5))
 (segment (start 142.5 78.685) (end 145.815 78.685) (width 1) (layer "F.Cu") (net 5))
 (segment (start 150.59 73.09) (end 150.274758 73.09) (width 0.5) (layer "F.Cu") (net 5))
 (segment (start 149.6 78.45) (end 146.05 78.45) (width 1) (layer "F.Cu") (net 5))
 (segment (start 153.4 78.45) (end 149.6 78.45) (width 1) (layer "F.Cu") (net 5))
 (segment (start 155.61 78.25) (end 156.5 79.14) (width 1) (layer "F.Cu") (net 5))
 (segment (start 145.815 78.685) (end 146 78.5) (width 1) (layer "F.Cu") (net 5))
 (segment (start 150.274758 73.09) (end 146.926 76.438758) (width 0.5) (layer "F.Cu") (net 5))
 (segment (start 146.926 76.438758) (end 146.926 77.574) (width 0.5) (layer "F.Cu") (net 5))
 (segment (start 149.6 78.45) (end 149.6 81.2) (width 0.5) (layer "F.Cu") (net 5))
 (segment (start 153.4 78.25) (end 155.61 78.25) (width 1) (layer "F.Cu") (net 5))
 (segment (start 150.45 82.05) (end 151.2 82.05) (width 0.5) (layer "F.Cu") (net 5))
 (segment (start 153.124 86.176) (end 153.3 86) (width 0.5) (layer "F.Cu") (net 2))
 (segment (start 142.5 81.685) (end 143.935 81.685) (width 0.5) (layer "F.Cu") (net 2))
 (segment (start 142.5 81.685) (end 143.747075 81.685) (width 0.5) (layer "F.Cu") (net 2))
 (segment (start 143.747075 81.685) (end 147.062075 85) (width 1) (layer "F.Cu") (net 2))
 (segment (start 159.5 83.5) (end 159.5 87.5) (width 0.2) (layer "F.Cu") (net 2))
 (segment (start 159.5 87.5) (end 158.4 88.6) (width 0.2) (layer "F.Cu") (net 2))
 (segment (start 149.5 85.725) (end 150.275 86.5) (width 1) (layer "F.Cu") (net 2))
 (segment (start 150.662075 88.6) (end 147.062075 85) (width 0.2) (layer "F.Cu") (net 2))
 (segment (start 150.275 86.5) (end 153.3 86.5) (width 1) (layer "F.Cu") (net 2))
 (segment (start 149.5 85) (end 149.5 85.725) (width 1) (layer "F.Cu") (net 2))
 (segment (start 147.062075 85) (end 149.5 85) (width 1) (layer "F.Cu") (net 2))
 (segment (start 158.4 88.6) (end 150.662075 88.6) (width 0.2) (layer "F.Cu") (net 2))
 (segment (start 147 73.225) (end 147.886 72.339) (width 0.5) (layer "F.Cu") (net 4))
 (segment (start 151.491 72.43) (end 151.4 72.339) (width 0.2) (layer "F.Cu") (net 4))
 (segment (start 142.5 72.685) (end 143.04 73.225) (width 0.5) (layer "F.Cu") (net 4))
 (segment (start 152.409 72.339) (end 155.659 72.339) (width 0.5) (layer "F.Cu") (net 4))
 (segment (start 150.59 76.91) (end 150.822 76.91) (width 0.2) (layer "F.Cu") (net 4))
 (segment (start 150.822 76.91) (end 151.491 76.241) (width 0.2) (layer "F.Cu") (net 4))
 (segment (start 151.4 72.339) (end 152.409 72.339) (width 0.5) (layer "F.Cu") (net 4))
 (segment (start 151.491 76.241) (end 151.491 72.43) (width 0.2) (layer "F.Cu") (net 4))
 (segment (start 155.659 72.339) (end 156.41 73.09) (width 0.5) (layer "F.Cu") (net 4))
 (segment (start 143.04 73.225) (end 147 73.225) (width 0.5) (layer "F.Cu") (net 4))
 (segment (start 147.886 72.339) (end 151.4 72.339) (width 0.5) (layer "F.Cu") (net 4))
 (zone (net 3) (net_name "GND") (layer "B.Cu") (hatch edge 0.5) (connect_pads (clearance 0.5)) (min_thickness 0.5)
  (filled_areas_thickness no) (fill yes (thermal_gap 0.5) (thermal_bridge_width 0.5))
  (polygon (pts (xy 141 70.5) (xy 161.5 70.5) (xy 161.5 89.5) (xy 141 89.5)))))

